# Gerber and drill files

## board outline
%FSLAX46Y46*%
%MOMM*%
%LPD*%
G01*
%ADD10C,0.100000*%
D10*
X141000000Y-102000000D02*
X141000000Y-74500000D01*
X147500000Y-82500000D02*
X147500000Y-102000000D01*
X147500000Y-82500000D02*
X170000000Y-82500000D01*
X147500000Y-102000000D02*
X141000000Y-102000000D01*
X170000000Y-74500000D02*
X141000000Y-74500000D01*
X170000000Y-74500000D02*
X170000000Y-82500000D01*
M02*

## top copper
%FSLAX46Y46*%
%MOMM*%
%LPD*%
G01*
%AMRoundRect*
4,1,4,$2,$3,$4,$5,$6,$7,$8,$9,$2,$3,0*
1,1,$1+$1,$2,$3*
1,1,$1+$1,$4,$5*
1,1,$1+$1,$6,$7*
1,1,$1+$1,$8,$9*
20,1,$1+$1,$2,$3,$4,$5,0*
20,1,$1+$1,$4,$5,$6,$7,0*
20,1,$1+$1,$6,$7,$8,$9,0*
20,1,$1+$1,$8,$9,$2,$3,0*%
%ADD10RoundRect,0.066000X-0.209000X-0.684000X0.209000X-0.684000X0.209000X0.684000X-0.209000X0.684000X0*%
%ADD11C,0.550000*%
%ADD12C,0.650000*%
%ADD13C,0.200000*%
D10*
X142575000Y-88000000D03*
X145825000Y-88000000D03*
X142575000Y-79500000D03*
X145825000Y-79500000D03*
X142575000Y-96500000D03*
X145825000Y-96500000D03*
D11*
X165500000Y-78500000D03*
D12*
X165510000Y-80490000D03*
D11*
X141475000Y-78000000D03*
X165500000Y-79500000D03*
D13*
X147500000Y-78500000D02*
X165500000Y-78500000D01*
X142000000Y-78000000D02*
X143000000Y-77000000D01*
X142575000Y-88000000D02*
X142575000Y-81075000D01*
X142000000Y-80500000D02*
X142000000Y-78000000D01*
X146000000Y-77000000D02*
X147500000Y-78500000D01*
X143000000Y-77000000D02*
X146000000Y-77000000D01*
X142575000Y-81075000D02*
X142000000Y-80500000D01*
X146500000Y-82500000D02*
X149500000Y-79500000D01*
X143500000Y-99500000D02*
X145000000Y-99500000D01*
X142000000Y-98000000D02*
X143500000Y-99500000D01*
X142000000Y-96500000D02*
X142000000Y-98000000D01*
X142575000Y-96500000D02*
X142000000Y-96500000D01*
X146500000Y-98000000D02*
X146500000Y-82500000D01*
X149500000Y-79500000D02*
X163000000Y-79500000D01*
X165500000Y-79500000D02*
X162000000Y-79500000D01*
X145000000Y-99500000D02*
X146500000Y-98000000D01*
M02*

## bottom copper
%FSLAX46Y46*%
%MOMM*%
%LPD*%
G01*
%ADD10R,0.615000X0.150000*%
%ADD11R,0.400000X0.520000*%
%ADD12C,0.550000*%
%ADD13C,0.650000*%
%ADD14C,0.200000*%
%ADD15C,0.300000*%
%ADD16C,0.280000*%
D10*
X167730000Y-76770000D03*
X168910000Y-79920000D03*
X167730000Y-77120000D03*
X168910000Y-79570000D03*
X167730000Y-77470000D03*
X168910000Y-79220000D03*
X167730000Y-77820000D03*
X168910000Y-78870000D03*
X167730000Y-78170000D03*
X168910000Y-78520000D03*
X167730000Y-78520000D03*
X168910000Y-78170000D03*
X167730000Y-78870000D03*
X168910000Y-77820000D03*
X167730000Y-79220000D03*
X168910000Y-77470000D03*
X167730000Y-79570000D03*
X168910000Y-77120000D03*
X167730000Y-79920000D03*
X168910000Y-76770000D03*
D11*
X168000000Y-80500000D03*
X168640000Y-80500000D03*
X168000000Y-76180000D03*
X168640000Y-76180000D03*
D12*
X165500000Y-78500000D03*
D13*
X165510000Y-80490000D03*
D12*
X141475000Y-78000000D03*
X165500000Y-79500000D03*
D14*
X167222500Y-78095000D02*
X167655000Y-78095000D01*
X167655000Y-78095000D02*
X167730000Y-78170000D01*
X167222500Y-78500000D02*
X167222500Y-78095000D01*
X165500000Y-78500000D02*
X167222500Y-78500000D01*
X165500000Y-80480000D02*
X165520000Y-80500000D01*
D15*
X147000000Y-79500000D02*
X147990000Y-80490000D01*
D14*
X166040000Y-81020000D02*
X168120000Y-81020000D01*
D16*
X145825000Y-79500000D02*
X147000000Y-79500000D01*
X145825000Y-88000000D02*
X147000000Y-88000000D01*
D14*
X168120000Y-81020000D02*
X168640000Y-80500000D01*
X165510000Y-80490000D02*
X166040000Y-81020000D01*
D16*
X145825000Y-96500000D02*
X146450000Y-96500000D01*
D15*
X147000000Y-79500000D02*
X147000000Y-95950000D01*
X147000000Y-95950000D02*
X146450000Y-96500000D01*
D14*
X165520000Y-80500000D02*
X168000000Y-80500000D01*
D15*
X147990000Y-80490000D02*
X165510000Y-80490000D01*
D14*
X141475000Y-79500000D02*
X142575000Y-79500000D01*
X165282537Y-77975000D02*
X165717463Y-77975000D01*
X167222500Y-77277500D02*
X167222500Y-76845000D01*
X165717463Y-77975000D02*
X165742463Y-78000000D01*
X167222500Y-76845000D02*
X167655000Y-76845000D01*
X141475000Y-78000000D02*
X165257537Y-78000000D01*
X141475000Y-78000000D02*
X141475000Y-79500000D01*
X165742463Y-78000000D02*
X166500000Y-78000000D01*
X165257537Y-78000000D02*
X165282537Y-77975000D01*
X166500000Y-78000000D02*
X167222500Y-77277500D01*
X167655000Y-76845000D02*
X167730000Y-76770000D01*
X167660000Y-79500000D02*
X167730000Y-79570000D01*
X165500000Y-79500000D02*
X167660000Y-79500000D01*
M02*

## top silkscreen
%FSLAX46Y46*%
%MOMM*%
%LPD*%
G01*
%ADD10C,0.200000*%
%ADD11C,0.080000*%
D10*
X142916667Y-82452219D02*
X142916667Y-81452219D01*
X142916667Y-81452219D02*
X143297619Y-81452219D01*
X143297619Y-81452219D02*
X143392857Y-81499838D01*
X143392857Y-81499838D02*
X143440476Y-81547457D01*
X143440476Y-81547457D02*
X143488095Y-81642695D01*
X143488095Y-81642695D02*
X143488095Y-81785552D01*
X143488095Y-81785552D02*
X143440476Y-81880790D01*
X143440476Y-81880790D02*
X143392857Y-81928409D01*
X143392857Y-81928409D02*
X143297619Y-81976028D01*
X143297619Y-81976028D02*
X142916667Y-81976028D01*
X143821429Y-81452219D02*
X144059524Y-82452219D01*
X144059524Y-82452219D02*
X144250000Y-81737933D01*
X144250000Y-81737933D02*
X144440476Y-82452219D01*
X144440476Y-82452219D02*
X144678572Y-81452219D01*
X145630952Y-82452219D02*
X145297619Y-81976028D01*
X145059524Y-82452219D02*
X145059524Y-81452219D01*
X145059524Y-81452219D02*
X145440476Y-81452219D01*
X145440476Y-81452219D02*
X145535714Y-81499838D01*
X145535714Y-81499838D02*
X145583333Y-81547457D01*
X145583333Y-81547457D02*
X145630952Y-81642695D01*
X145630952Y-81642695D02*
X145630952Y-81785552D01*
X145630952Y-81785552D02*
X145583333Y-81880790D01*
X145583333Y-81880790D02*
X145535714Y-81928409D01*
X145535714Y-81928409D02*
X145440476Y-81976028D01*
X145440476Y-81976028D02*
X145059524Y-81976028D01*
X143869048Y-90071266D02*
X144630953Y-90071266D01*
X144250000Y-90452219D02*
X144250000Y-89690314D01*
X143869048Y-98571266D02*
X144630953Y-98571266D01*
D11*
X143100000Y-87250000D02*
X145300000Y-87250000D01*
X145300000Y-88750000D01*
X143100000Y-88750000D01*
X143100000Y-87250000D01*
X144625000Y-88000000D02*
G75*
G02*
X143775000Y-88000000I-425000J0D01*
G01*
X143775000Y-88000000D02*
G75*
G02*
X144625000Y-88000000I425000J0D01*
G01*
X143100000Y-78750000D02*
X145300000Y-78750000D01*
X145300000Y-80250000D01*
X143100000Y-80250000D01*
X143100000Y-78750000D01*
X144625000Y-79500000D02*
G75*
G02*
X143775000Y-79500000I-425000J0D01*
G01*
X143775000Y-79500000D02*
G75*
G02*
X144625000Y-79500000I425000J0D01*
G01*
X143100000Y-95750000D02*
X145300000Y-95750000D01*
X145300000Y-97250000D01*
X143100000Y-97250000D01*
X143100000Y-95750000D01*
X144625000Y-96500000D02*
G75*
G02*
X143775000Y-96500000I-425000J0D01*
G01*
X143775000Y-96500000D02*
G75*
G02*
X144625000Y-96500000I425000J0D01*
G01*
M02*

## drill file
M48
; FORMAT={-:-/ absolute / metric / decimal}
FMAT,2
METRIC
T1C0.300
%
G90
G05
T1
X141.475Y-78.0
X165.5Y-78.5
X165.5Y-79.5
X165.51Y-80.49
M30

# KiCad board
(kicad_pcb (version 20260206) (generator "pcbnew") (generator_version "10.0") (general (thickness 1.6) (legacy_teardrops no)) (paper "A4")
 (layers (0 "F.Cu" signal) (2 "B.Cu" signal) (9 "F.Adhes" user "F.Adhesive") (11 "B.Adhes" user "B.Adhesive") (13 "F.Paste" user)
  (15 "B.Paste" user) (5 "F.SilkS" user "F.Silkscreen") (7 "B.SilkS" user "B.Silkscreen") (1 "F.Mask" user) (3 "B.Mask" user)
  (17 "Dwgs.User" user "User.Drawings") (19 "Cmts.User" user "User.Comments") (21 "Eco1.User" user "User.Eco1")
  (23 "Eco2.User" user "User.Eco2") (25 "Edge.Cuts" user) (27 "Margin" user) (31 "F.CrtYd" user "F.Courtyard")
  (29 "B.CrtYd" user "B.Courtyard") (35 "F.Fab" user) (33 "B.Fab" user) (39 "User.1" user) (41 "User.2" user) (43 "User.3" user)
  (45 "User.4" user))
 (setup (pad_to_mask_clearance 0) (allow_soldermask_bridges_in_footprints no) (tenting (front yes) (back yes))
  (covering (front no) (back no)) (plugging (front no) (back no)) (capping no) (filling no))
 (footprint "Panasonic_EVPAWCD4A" (layer "F.Cu") (at 144.2 88)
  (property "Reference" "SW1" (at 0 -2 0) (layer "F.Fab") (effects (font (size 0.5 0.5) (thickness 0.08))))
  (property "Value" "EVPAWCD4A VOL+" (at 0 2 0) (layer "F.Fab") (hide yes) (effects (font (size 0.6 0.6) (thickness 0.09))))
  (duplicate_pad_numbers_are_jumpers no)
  (fp_rect (start -1.1 -0.75) (end 1.1 0.75) (stroke (width 0.08) (type solid)) (fill no) (layer "F.SilkS"))
  (fp_circle (center 0 0) (end 0.425 0) (stroke (width 0.08) (type solid)) (fill no) (layer "F.SilkS"))
  (pad "1" smd roundrect (at -1.625 0) (size 0.55 1.5) (layers "F.Cu" "F.Mask" "F.Paste") (roundrect_rratio 0.12) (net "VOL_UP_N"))
  (pad "2" smd roundrect (at 1.625 0) (size 0.55 1.5) (layers "F.Cu" "F.Mask" "F.Paste") (roundrect_rratio 0.12) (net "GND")))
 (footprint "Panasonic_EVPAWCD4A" (layer "F.Cu") (at 144.2 79.5)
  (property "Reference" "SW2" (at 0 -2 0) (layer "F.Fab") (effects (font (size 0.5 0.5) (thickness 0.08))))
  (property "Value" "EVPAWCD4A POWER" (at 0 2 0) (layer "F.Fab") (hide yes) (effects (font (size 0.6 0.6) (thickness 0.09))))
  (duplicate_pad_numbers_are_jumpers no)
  (fp_rect (start -1.1 -0.75) (end 1.1 0.75) (stroke (width 0.08) (type solid)) (fill no) (layer "F.SilkS"))
  (fp_circle (center 0 0) (end 0.425 0) (stroke (width 0.08) (type solid)) (fill no) (layer "F.SilkS"))
  (pad "1" smd roundrect (at -1.625 0) (size 0.55 1.5) (layers "F.Cu" "F.Mask" "F.Paste") (roundrect_rratio 0.12) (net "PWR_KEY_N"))
  (pad "2" smd roundrect (at 1.625 0) (size 0.55 1.5) (layers "F.Cu" "F.Mask" "F.Paste") (roundrect_rratio 0.12) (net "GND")))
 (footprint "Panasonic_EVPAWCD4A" (layer "F.Cu") (at 144.2 96.5)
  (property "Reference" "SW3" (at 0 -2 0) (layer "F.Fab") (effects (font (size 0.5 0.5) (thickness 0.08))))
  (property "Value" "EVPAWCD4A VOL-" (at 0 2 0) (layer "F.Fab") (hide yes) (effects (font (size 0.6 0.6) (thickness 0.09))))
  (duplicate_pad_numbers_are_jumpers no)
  (fp_rect (start -1.1 -0.75) (end 1.1 0.75) (stroke (width 0.08) (type solid)) (fill no) (layer "F.SilkS"))
  (fp_circle (center 0 0) (end 0.425 0) (stroke (width 0.08) (type solid)) (fill no) (layer "F.SilkS"))
  (pad "1" smd roundrect (at -1.625 0) (size 0.55 1.5) (layers "F.Cu" "F.Mask" "F.Paste") (roundrect_rratio 0.12) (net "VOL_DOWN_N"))
  (pad "2" smd roundrect (at 1.625 0) (size 0.55 1.5) (layers "F.Cu" "F.Mask" "F.Paste") (roundrect_rratio 0.12) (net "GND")))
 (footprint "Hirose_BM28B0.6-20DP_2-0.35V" (layer "B.Cu") (at 168.32 78.34 90)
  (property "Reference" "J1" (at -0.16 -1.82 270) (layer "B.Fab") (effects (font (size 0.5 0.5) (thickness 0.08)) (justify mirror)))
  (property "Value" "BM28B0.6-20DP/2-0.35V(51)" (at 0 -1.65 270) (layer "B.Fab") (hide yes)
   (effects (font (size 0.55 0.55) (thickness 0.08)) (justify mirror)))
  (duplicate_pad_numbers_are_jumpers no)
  (pad "1" smd rect (at 1.57 -0.59 90) (size 0.15 0.615) (layers "B.Cu" "B.Mask" "B.Paste") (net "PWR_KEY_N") (clearance 0.08))
  (pad "2" smd rect (at -1.58 0.59 90) (size 0.15 0.615) (layers "B.Cu" "B.Mask" "B.Paste") (clearance 0.08))
  (pad "3" smd rect (at 1.22 -0.59 90) (size 0.15 0.615) (layers "B.Cu" "B.Mask" "B.Paste") (clearance 0.08))
  (pad "4" smd rect (at -1.23 0.59 90) (size 0.15 0.615) (layers "B.Cu" "B.Mask" "B.Paste") (clearance 0.08))
  (pad "5" smd rect (at 0.87 -0.59 90) (size 0.15 0.615) (layers "B.Cu" "B.Mask" "B.Paste") (clearance 0.08))
  (pad "6" smd rect (at -0.88 0.59 90) (size 0.15 0.615) (layers "B.Cu" "B.Mask" "B.Paste") (clearance 0.08))
  (pad "7" smd rect (at 0.52 -0.59 90) (size 0.15 0.615) (layers "B.Cu" "B.Mask" "B.Paste") (clearance 0.08))
  (pad "8" smd rect (at -0.53 0.59 90) (size 0.15 0.615) (layers "B.Cu" "B.Mask" "B.Paste") (clearance 0.08))
  (pad "9" smd rect (at 0.17 -0.59 90) (size 0.15 0.615) (layers "B.Cu" "B.Mask" "B.Paste") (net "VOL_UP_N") (clearance 0.08))
  (pad "10" smd rect (at -0.18 0.59 90) (size 0.15 0.615) (layers "B.Cu" "B.Mask" "B.Paste") (clearance 0.08))
  (pad "11" smd rect (at -0.18 -0.59 90) (size 0.15 0.615) (layers "B.Cu" "B.Mask" "B.Paste") (clearance 0.08))
  (pad "12" smd rect (at 0.17 0.59 90) (size 0.15 0.615) (layers "B.Cu" "B.Mask" "B.Paste") (clearance 0.08))
  (pad "13" smd rect (at -0.53 -0.59 90) (size 0.15 0.615) (layers "B.Cu" "B.Mask" "B.Paste") (clearance 0.08))
  (pad "14" smd rect (at 0.52 0.59 90) (size 0.15 0.615) (layers "B.Cu" "B.Mask" "B.Paste") (clearance 0.08))
  (pad "15" smd rect (at -0.88 -0.59 90) (size 0.15 0.615) (layers "B.Cu" "B.Mask" "B.Paste") (clearance 0.08))
  (pad "16" smd rect (at 0.87 0.59 90) (size 0.15 0.615) (layers "B.Cu" "B.Mask" "B.Paste") (clearance 0.08))
  (pad "17" smd rect (at -1.23 -0.59 90) (size 0.15 0.615) (layers "B.Cu" "B.Mask" "B.Paste") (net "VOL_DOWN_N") (clearance 0.08))
  (pad "18" smd rect (at 1.22 0.59 90) (size 0.15 0.615) (layers "B.Cu" "B.Mask" "B.Paste") (clearance 0.08))
  (pad "19" smd rect (at -1.58 -0.59 90) (size 0.15 0.615) (layers "B.Cu" "B.Mask" "B.Paste") (clearance 0.08))
  (pad "20" smd rect (at 1.57 0.59 90) (size 0.15 0.615) (layers "B.Cu" "B.Mask" "B.Paste") (clearance 0.08))
  (pad "21" smd rect (at -2.16 -0.32 90) (size 0.52 0.4) (layers "B.Cu" "B.Mask" "B.Paste") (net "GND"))
  (pad "21" smd rect (at -2.16 0.32 90) (size 0.52 0.4) (layers "B.Cu" "B.Mask" "B.Paste") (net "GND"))
  (pad "22" smd rect (at 2.16 -0.32 90) (size 0.52 0.4) (layers "B.Cu" "B.Mask" "B.Paste"))
  (pad "22" smd rect (at 2.16 0.32 90) (size 0.52 0.4) (layers "B.Cu" "B.Mask" "B.Paste")))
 (gr_line (start 141 102) (end 141 74.5) (stroke (width 0.1) (type default)) (layer "Edge.Cuts"))
 (gr_line (start 147.5 82.5) (end 147.5 102) (stroke (width 0.1) (type default)) (layer "Edge.Cuts"))
 (gr_line (start 147.5 82.5) (end 170 82.5) (stroke (width 0.1) (type default)) (layer "Edge.Cuts"))
 (gr_line (start 147.5 102) (end 141 102) (stroke (width 0.1) (type default)) (layer "Edge.Cuts"))
 (gr_line (start 170 74.5) (end 141 74.5) (stroke (width 0.1) (type default)) (layer "Edge.Cuts"))
 (gr_line (start 170 74.5) (end 170 82.5) (stroke (width 0.1) (type default)) (layer "Edge.Cuts"))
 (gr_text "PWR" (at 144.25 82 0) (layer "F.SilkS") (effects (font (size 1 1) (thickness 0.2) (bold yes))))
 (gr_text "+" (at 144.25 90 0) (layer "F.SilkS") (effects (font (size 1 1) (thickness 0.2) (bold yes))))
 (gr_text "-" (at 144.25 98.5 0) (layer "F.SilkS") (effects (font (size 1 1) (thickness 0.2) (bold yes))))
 (segment (start 147.5 78.5) (end 165.5 78.5) (width 0.2) (layer "F.Cu") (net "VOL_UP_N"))
 (segment (start 142 78) (end 143 77) (width 0.2) (layer "F.Cu") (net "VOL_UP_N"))
 (segment (start 142.575 88) (end 142.575 81.075) (width 0.2) (layer "F.Cu") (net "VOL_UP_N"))
 (segment (start 142 80.5) (end 142 78) (width 0.2) (layer "F.Cu") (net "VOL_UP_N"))
 (segment (start 146 77) (end 147.5 78.5) (width 0.2) (layer "F.Cu") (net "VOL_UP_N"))
 (segment (start 143 77) (end 146 77) (width 0.2) (layer "F.Cu") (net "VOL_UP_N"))
 (segment (start 142.575 81.075) (end 142 80.5) (width 0.2) (layer "F.Cu") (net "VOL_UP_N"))
 (via (at 165.5 78.5) (size 0.55) (drill 0.3) (layers "F.Cu" "B.Cu") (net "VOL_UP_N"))
 (segment (start 167.2225 78.095) (end 167.655 78.095) (width 0.2) (layer "B.Cu") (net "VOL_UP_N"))
 (segment (start 167.655 78.095) (end 167.73 78.17) (width 0.2) (layer "B.Cu") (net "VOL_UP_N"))
 (segment (start 167.2225 78.5) (end 167.2225 78.095) (width 0.2) (layer "B.Cu") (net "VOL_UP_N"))
 (segment (start 165.5 78.5) (end 167.2225 78.5) (width 0.2) (layer "B.Cu") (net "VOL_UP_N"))
 (via (at 165.51 80.49) (size 0.65) (drill 0.3) (layers "F.Cu" "B.Cu") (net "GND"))
 (segment (start 165.5 80.48) (end 165.52 80.5) (width 0.2) (layer "B.Cu") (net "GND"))
 (segment (start 147 79.5) (end 147.99 80.49) (width 0.3) (layer "B.Cu") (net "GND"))
 (segment (start 166.04 81.02) (end 168.12 81.02) (width 0.2) (layer "B.Cu") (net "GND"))
 (segment (start 145.825 79.5) (end 147 79.5) (width 0.28) (layer "B.Cu") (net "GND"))
 (segment (start 145.825 88) (end 147 88) (width 0.28) (layer "B.Cu") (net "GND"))
 (segment (start 168.12 81.02) (end 168.64 80.5) (width 0.2) (layer "B.Cu") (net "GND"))
 (segment (start 165.51 80.49) (end 166.04 81.02) (width 0.2) (layer "B.Cu") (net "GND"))
 (segment (start 145.825 96.5) (end 146.45 96.5) (width 0.28) (layer "B.Cu") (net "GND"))
 (segment (start 147 79.5) (end 147 95.95) (width 0.3) (layer "B.Cu") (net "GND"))
 (segment (start 147 95.95) (end 146.45 96.5) (width 0.3) (layer "B.Cu") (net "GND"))
 (segment (start 165.52 80.5) (end 168 80.5) (width 0.2) (layer "B.Cu") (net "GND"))
 (segment (start 147.99 80.49) (end 165.51 80.49) (width 0.3) (layer "B.Cu") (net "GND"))
 (via (at 141.475 78) (size 0.55) (drill 0.3) (layers "F.Cu" "B.Cu") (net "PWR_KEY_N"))
 (segment (start 141.475 79.5) (end 142.575 79.5) (width 0.2) (layer "B.Cu") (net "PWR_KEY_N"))
 (segment (start 165.282537 77.975) (end 165.717463 77.975) (width 0.2) (layer "B.Cu") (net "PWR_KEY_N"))
 (segment (start 167.2225 77.2775) (end 167.2225 76.845) (width 0.2) (layer "B.Cu") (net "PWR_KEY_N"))
 (segment (start 165.717463 77.975) (end 165.742463 78) (width 0.2) (layer "B.Cu") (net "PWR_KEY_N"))
 (segment (start 167.2225 76.845) (end 167.655 76.845) (width 0.2) (layer "B.Cu") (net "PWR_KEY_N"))
 (segment (start 141.475 78) (end 165.257537 78) (width 0.2) (layer "B.Cu") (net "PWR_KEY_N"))
 (segment (start 141.475 78) (end 141.475 79.5) (width 0.2) (layer "B.Cu") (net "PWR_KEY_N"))
 (segment (start 165.742463 78) (end 166.5 78) (width 0.2) (layer "B.Cu") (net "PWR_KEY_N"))
 (segment (start 165.257537 78) (end 165.282537 77.975) (width 0.2) (layer "B.Cu") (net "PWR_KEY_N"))
 (segment (start 166.5 78) (end 167.2225 77.2775) (width 0.2) (layer "B.Cu") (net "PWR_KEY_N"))
 (segment (start 167.655 76.845) (end 167.73 76.77) (width 0.2) (layer "B.Cu") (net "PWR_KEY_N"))
 (segment (start 146.5 82.5) (end 149.5 79.5) (width 0.2) (layer "F.Cu") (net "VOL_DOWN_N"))
 (segment (start 143.5 99.5) (end 145 99.5) (width 0.2) (layer "F.Cu") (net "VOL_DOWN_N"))
 (segment (start 142 98) (end 143.5 99.5) (width 0.2) (layer "F.Cu") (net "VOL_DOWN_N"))
 (segment (start 142 96.5) (end 142 98) (width 0.2) (layer "F.Cu") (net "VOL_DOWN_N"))
 (segment (start 142.575 96.5) (end 142 96.5) (width 0.2) (layer "F.Cu") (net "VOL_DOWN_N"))
 (segment (start 146.5 98) (end 146.5 82.5) (width 0.2) (layer "F.Cu") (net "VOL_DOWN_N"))
 (segment (start 149.5 79.5) (end 163 79.5) (width 0.2) (layer "F.Cu") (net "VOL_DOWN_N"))
 (segment (start 165.5 79.5) (end 162 79.5) (width 0.2) (layer "F.Cu") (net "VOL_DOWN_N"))
 (segment (start 145 99.5) (end 146.5 98) (width 0.2) (layer "F.Cu") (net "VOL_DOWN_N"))
 (via (at 165.5 79.5) (size 0.55) (drill 0.3) (layers "F.Cu" "B.Cu") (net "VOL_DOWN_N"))
 (segment (start 167.66 79.5) (end 167.73 79.57) (width 0.2) (layer "B.Cu") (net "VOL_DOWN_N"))
 (segment (start 165.5 79.5) (end 167.66 79.5) (width 0.2) (layer "B.Cu") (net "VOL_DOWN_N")))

